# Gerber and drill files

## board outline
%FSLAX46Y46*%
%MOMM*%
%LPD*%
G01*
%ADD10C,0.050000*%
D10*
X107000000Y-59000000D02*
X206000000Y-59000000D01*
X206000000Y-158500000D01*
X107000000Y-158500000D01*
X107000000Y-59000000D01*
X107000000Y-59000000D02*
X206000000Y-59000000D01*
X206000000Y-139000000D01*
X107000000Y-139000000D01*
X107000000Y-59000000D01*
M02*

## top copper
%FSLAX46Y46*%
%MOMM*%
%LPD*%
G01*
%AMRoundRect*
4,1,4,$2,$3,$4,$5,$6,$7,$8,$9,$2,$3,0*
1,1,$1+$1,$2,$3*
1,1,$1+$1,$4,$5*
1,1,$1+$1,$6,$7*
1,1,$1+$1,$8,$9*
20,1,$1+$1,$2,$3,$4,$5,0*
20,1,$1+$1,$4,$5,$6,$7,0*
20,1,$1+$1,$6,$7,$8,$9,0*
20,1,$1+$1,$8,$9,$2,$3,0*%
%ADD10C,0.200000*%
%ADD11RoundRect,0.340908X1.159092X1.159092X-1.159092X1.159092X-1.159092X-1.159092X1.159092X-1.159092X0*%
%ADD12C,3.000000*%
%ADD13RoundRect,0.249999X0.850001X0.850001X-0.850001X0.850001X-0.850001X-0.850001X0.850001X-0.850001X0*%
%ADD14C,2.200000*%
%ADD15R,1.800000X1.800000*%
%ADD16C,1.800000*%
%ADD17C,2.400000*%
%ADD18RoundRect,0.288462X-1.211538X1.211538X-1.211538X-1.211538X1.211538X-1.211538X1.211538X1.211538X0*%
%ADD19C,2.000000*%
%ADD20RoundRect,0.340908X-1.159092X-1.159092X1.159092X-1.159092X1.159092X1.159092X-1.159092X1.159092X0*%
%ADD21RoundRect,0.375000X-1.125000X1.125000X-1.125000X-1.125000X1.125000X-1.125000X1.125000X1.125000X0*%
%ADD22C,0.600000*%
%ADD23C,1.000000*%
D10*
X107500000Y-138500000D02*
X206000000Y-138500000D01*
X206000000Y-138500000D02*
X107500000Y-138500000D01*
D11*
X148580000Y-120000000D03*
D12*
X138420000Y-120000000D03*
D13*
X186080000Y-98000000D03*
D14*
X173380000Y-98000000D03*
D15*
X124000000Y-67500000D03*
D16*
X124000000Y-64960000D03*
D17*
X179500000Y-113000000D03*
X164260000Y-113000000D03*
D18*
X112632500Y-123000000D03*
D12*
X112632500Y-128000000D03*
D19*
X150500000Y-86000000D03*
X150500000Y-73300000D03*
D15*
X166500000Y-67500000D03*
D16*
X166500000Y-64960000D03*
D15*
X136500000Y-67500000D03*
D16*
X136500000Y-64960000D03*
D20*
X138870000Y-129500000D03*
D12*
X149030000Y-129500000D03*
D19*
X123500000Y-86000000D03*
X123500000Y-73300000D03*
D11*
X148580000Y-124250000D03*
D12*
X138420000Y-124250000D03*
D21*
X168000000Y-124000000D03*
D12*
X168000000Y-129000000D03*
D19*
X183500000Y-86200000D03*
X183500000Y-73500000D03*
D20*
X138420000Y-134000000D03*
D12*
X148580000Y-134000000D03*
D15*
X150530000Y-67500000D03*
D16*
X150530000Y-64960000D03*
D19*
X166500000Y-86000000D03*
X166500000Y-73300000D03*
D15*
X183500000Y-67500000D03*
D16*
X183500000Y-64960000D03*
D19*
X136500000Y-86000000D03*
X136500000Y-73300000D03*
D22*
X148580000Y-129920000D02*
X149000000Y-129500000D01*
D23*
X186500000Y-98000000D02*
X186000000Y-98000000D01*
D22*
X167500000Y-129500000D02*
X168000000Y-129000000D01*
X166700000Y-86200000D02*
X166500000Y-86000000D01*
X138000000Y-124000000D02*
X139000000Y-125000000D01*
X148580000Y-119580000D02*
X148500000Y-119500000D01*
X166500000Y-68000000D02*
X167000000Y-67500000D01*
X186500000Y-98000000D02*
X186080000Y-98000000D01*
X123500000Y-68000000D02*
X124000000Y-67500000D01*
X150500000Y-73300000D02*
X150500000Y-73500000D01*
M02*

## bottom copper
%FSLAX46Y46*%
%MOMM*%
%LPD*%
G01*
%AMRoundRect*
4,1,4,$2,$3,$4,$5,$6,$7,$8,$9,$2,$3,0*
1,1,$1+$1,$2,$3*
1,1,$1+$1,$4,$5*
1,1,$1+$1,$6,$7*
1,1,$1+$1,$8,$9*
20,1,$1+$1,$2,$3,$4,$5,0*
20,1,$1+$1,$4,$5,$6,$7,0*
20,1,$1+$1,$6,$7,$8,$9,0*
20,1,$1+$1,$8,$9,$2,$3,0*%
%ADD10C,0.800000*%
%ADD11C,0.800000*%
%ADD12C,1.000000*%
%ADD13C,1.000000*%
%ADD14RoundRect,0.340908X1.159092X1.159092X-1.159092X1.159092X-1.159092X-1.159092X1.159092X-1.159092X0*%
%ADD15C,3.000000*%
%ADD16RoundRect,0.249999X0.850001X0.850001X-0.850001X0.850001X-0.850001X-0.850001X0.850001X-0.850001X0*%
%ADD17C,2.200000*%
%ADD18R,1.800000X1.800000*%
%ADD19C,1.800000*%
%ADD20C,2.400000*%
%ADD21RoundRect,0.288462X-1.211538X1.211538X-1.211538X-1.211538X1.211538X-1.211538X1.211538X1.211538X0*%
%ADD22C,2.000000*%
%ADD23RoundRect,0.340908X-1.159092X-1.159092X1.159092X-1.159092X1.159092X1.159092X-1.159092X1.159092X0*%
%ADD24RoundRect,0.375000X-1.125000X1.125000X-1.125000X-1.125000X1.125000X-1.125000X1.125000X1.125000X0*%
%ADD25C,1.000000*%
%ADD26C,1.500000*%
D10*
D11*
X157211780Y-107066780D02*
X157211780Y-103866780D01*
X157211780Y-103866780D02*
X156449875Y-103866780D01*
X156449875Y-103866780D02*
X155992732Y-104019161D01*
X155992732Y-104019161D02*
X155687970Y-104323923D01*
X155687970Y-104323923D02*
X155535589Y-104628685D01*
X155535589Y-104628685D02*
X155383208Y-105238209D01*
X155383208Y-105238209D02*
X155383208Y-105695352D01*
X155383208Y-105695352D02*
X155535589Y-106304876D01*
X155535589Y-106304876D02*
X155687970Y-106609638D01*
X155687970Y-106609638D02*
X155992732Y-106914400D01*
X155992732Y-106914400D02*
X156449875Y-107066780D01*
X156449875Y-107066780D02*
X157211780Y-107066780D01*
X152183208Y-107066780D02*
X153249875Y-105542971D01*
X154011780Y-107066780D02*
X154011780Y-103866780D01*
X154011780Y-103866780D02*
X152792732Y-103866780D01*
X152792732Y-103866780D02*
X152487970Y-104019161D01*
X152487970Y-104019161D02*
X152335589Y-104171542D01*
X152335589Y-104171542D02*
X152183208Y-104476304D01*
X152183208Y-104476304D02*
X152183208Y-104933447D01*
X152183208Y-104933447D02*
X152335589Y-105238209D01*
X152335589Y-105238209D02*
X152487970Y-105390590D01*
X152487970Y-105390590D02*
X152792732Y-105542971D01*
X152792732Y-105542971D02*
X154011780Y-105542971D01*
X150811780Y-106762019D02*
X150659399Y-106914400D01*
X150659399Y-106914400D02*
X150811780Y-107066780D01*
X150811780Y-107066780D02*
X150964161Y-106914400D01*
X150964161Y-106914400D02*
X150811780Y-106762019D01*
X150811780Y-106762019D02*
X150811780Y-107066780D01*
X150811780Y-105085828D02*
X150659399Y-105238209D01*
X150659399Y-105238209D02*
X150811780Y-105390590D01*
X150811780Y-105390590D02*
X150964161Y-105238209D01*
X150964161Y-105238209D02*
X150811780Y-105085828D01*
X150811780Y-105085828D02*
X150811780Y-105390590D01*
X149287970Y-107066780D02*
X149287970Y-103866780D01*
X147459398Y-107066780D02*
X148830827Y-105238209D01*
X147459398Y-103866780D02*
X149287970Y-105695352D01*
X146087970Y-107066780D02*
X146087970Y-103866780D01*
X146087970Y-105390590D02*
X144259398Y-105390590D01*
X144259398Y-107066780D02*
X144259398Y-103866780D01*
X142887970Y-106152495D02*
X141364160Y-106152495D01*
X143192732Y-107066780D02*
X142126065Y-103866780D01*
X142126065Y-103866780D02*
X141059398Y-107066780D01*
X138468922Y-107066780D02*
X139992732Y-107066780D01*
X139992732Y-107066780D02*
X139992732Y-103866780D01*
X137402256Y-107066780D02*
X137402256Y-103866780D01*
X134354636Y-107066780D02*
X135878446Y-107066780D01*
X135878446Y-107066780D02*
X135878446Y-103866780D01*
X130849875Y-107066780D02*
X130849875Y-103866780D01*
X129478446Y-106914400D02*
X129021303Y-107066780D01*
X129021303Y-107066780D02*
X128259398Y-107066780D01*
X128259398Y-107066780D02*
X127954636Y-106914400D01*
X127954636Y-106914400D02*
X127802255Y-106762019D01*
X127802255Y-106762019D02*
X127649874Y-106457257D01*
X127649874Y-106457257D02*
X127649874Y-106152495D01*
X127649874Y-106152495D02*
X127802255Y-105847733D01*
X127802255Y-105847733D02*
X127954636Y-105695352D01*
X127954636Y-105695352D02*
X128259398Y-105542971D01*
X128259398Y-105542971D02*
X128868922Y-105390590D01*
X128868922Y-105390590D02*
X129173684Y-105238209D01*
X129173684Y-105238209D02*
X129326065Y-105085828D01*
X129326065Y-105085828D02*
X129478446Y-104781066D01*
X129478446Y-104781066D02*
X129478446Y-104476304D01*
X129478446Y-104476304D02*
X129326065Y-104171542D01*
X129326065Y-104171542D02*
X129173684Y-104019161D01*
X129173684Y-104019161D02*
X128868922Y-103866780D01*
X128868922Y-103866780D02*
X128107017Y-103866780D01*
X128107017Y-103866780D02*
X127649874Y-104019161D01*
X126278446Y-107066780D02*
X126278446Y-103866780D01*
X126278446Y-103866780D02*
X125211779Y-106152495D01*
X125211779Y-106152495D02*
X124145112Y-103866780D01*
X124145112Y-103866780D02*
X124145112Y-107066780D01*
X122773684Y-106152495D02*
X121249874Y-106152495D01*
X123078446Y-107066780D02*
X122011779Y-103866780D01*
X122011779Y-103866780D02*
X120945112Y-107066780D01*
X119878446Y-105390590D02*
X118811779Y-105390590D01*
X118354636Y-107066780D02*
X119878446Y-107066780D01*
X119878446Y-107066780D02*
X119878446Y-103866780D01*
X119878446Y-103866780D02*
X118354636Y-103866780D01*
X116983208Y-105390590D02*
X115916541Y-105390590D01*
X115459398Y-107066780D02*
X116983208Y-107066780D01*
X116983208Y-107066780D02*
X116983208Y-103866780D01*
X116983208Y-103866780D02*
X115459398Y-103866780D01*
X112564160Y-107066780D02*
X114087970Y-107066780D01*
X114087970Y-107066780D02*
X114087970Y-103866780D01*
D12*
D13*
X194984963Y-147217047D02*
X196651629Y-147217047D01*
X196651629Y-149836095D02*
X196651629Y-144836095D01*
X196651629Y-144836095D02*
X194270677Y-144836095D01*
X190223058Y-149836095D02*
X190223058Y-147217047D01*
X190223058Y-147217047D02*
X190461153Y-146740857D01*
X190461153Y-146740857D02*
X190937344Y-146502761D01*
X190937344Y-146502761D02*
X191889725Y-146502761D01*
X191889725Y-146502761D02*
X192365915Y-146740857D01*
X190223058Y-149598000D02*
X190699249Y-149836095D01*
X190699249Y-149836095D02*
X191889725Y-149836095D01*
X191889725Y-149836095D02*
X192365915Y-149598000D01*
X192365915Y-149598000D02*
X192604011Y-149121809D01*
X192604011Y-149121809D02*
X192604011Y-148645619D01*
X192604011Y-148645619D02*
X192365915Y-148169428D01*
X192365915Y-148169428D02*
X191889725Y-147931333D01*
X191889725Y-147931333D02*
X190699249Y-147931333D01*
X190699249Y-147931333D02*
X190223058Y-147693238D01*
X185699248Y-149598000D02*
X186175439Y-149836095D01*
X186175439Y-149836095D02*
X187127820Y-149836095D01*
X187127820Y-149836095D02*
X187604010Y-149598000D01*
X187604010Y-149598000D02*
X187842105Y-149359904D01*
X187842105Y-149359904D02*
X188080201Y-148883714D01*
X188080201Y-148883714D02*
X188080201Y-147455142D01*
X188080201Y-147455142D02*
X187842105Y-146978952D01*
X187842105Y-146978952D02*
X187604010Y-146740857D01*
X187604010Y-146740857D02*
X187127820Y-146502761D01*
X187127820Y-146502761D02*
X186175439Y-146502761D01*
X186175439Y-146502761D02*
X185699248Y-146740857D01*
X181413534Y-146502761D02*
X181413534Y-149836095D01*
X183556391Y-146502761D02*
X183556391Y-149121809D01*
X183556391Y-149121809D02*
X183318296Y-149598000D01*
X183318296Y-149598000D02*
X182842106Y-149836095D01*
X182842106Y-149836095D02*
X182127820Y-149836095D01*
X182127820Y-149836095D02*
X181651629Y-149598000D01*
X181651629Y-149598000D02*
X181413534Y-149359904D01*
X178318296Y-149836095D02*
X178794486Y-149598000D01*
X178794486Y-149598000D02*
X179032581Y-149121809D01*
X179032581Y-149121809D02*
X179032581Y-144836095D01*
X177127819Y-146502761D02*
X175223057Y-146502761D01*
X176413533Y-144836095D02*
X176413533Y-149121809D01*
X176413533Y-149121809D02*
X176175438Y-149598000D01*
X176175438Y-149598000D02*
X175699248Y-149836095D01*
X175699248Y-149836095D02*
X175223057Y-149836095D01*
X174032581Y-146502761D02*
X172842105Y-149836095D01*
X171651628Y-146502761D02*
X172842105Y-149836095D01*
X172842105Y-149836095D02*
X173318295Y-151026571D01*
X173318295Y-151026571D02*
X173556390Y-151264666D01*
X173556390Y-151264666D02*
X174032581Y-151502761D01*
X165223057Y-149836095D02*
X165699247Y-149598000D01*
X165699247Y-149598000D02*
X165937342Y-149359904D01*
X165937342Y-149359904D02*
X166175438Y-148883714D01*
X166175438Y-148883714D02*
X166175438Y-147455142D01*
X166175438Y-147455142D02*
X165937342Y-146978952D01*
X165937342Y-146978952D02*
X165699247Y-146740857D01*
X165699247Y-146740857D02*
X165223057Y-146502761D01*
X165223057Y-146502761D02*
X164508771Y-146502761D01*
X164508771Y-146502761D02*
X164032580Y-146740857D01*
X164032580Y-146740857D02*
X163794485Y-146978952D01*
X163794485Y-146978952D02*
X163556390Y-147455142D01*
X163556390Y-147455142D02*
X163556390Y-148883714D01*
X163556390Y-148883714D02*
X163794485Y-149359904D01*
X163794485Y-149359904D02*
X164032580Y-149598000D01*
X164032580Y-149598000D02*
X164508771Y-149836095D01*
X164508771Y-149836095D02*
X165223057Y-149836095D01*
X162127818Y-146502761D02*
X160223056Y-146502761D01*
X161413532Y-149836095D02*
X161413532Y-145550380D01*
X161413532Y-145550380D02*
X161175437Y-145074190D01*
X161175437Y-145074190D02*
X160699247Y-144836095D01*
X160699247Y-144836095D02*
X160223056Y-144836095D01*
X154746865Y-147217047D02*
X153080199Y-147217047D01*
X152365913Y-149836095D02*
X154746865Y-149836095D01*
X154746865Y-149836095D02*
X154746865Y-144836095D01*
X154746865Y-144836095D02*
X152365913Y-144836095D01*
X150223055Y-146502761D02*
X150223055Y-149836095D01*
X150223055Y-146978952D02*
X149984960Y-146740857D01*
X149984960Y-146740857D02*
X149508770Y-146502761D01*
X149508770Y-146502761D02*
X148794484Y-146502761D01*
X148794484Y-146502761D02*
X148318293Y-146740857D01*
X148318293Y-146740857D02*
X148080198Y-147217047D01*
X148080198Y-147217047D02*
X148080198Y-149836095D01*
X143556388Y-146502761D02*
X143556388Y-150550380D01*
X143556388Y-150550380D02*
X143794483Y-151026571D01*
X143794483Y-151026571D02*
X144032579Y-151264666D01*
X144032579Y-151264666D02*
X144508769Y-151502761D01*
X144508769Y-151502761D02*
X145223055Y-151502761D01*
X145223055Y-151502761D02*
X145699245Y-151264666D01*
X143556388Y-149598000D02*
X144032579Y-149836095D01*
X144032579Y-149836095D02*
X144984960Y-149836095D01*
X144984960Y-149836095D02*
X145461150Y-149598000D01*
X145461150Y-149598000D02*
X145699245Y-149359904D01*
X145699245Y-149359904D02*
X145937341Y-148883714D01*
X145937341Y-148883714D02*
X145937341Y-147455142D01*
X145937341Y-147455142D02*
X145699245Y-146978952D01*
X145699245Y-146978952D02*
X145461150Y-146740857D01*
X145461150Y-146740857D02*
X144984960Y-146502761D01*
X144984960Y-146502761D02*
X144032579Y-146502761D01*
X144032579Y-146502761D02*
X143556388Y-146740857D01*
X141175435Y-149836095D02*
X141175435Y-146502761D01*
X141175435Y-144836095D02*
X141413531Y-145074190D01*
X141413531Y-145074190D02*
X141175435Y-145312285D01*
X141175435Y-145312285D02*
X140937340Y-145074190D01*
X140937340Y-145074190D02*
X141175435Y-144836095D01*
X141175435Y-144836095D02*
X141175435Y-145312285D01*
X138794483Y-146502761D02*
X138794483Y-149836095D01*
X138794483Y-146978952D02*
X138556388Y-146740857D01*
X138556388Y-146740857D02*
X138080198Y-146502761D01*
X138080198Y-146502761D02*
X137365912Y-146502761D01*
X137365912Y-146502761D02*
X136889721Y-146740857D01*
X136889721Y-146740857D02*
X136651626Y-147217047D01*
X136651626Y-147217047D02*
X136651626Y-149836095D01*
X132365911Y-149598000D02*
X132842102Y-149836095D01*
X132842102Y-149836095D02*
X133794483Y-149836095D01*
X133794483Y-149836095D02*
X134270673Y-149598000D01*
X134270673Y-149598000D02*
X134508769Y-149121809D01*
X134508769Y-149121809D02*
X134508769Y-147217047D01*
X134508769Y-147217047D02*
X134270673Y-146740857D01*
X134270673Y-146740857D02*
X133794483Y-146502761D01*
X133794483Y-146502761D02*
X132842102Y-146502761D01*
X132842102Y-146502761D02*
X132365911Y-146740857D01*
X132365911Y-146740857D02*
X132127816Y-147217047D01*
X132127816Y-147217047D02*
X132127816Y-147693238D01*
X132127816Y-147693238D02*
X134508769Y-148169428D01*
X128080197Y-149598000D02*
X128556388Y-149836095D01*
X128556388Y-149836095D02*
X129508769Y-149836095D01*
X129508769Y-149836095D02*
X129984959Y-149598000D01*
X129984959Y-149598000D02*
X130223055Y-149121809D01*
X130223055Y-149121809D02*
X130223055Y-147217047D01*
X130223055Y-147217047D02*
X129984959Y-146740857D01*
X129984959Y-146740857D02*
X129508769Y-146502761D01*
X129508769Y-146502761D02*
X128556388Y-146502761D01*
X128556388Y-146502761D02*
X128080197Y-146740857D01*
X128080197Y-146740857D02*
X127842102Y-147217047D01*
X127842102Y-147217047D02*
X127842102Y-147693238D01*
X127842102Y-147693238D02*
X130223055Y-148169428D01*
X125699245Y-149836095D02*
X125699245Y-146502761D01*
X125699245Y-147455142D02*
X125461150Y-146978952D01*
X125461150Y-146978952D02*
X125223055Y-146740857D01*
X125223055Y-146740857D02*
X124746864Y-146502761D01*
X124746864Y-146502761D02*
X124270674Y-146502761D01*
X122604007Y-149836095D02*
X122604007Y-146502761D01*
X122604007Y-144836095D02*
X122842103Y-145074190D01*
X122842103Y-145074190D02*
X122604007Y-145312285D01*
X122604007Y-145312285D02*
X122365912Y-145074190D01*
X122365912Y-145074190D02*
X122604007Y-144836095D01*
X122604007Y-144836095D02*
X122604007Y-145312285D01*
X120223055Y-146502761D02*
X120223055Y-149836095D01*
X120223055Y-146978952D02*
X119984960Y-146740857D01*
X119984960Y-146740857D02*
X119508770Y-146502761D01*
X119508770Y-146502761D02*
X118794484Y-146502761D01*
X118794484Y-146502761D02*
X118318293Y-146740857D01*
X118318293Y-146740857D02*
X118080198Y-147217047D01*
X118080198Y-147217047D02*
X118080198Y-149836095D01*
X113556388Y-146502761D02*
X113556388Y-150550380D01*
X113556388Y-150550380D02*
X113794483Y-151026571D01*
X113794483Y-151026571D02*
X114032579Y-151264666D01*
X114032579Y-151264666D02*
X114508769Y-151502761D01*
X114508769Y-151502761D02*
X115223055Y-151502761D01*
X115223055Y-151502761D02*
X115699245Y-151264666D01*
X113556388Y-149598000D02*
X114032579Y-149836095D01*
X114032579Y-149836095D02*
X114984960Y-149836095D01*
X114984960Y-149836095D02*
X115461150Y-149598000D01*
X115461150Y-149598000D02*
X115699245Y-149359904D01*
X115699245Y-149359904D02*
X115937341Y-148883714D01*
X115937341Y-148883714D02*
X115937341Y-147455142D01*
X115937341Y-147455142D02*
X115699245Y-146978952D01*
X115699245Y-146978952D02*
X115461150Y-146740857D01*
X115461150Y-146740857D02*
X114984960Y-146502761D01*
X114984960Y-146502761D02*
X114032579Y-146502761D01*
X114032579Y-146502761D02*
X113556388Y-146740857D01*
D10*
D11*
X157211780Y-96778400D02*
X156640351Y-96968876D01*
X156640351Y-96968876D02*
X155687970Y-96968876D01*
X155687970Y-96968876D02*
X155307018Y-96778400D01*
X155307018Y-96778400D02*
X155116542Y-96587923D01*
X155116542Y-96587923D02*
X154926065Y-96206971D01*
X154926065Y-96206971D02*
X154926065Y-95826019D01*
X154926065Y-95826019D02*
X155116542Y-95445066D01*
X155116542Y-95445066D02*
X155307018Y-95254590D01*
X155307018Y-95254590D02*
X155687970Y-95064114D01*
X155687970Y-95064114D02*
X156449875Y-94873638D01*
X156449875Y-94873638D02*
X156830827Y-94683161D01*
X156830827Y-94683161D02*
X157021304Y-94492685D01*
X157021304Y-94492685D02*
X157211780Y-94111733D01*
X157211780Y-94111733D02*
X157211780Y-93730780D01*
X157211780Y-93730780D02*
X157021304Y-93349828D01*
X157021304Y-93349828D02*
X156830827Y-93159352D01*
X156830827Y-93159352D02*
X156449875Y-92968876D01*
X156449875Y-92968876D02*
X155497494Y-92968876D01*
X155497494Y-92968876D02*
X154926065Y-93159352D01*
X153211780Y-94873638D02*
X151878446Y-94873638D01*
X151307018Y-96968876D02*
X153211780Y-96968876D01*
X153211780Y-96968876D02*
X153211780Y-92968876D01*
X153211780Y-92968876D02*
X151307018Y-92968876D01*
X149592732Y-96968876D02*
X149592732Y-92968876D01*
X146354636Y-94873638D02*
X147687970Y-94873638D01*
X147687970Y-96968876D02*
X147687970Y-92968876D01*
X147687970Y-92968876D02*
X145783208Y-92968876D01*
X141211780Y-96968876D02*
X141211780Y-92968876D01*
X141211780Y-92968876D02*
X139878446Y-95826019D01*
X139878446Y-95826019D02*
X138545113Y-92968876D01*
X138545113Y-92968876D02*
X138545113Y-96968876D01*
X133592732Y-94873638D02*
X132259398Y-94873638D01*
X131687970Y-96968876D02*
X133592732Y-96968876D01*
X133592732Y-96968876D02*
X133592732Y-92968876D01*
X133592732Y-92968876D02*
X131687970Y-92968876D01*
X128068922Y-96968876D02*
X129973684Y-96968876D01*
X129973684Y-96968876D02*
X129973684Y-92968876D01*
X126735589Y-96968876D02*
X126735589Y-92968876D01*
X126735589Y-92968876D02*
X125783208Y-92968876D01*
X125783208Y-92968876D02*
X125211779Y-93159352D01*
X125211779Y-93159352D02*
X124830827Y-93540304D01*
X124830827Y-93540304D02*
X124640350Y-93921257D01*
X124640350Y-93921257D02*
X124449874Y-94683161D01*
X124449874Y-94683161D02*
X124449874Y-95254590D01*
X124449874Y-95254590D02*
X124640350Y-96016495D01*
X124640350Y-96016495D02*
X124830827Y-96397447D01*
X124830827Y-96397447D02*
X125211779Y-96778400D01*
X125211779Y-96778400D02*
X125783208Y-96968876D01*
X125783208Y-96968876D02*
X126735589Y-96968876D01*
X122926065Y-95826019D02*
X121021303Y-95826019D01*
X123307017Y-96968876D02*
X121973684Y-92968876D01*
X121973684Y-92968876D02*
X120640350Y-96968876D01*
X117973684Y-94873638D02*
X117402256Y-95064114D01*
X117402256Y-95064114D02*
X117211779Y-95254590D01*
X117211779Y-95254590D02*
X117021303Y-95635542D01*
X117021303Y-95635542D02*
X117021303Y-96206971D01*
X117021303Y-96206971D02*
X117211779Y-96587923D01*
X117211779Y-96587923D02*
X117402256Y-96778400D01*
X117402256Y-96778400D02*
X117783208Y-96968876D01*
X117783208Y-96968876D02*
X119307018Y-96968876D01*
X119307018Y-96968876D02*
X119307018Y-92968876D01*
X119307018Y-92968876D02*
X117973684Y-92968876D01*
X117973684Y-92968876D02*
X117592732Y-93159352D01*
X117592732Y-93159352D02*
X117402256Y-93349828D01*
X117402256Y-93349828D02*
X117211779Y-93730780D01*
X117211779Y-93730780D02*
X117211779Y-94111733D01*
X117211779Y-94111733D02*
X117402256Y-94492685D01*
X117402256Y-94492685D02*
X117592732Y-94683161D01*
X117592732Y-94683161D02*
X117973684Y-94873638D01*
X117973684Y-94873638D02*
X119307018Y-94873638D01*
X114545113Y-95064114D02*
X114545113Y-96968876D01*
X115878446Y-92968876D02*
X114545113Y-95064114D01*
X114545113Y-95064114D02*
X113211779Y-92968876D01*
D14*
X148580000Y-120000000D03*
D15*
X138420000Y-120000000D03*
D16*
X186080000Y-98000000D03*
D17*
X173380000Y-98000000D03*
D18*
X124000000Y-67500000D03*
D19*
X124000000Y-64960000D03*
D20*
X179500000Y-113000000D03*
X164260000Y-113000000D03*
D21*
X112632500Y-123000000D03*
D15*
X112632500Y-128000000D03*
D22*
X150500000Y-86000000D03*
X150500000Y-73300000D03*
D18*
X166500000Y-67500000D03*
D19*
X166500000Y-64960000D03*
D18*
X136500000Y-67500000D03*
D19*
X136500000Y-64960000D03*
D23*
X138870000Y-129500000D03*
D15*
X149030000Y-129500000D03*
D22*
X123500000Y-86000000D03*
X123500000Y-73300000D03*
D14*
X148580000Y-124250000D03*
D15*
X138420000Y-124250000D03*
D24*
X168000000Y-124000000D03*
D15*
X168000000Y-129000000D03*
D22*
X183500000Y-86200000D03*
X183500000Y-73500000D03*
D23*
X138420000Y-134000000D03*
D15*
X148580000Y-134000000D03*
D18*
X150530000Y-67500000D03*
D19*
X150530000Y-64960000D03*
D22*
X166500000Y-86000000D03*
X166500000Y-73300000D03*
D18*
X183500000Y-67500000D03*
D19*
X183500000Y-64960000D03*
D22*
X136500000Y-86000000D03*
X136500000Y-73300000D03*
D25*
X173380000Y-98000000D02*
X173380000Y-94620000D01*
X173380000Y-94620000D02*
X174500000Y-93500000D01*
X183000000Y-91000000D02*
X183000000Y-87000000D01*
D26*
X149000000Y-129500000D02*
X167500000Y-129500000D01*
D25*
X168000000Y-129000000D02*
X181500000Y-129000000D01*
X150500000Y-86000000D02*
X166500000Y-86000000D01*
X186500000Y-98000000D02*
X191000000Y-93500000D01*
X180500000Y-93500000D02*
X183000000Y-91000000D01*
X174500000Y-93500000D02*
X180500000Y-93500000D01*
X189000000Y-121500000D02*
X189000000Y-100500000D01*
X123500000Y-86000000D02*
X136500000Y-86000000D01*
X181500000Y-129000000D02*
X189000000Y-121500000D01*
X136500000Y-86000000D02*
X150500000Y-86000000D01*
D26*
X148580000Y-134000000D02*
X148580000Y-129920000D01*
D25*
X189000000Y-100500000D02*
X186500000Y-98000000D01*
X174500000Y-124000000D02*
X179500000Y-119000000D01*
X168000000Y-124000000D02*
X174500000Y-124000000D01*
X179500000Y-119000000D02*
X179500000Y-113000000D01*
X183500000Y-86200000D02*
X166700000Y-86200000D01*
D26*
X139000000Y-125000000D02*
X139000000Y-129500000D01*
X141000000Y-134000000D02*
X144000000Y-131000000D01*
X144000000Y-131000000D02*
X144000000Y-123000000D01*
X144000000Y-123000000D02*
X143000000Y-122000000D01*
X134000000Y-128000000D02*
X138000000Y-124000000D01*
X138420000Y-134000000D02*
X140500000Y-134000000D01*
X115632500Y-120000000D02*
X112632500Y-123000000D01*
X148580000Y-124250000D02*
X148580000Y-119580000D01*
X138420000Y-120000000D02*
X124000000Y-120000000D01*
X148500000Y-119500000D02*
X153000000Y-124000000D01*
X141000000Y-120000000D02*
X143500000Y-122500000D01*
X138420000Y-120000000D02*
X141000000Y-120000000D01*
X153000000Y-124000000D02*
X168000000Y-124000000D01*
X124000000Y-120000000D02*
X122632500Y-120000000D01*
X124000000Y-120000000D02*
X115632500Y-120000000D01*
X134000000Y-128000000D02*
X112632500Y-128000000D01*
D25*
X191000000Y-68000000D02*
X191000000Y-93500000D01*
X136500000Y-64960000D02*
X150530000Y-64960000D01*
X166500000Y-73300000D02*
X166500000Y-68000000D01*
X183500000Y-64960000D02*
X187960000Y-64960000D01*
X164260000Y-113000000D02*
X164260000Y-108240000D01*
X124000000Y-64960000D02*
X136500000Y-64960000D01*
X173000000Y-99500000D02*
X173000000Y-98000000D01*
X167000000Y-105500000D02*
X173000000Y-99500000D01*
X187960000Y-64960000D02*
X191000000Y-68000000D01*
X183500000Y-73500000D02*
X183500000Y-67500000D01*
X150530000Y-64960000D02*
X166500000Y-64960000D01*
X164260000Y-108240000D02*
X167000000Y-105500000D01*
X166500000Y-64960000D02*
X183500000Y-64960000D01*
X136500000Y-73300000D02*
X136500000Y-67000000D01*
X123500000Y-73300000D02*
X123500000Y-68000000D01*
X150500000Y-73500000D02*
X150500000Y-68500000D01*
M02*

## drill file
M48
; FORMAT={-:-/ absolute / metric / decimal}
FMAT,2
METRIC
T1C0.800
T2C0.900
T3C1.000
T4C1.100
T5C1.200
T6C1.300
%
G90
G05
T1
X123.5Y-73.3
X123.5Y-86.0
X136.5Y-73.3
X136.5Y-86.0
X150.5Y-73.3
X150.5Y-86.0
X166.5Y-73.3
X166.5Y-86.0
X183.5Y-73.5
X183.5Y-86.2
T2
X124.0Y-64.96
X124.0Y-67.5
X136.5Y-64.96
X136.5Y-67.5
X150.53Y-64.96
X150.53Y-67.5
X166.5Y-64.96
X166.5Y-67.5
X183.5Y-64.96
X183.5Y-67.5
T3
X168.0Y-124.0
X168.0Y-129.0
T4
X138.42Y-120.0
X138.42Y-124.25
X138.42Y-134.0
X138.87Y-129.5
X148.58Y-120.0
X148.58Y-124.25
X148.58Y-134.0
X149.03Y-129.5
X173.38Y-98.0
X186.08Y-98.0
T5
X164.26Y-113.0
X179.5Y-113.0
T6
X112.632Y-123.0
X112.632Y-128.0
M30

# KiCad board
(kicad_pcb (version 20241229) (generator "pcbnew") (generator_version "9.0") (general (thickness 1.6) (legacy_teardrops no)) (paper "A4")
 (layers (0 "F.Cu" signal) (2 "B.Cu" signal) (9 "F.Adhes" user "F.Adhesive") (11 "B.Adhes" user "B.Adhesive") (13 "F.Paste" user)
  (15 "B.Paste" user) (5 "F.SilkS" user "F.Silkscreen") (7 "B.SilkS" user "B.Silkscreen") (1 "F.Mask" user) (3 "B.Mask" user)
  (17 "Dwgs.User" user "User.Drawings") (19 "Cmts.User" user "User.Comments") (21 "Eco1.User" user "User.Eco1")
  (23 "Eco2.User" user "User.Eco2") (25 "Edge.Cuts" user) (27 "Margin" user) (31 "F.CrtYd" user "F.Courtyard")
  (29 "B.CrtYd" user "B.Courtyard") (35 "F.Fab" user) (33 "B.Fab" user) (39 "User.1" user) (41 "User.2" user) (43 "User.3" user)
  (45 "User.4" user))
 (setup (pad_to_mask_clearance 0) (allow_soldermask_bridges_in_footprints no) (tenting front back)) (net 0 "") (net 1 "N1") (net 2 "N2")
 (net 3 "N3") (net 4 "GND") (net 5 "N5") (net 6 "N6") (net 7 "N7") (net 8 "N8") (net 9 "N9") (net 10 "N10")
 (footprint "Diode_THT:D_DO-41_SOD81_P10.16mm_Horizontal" (layer "F.Cu") (at 148.58 120 180)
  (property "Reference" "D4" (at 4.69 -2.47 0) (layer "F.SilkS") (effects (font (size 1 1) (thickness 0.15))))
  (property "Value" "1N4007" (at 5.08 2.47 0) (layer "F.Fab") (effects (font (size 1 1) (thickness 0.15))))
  (pad "1" thru_hole roundrect (at 0 0 180) (size 3 3) (drill 1.1) (layers "*.Cu" "*.Mask") (remove_unused_layers no)
   (roundrect_rratio 0.113636) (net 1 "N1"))
  (pad "2" thru_hole circle (at 10.16 0 180) (size 3 3) (drill 1.1) (layers "*.Cu" "*.Mask") (remove_unused_layers no) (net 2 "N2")))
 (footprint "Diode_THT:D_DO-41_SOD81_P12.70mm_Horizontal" (layer "F.Cu") (at 186.08 98 180)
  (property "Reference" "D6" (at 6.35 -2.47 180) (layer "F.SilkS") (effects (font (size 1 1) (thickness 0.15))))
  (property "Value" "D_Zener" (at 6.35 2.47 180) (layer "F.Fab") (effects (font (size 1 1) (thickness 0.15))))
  (pad "1" thru_hole roundrect (at 0 0 180) (size 2.2 2.2) (drill 1.1) (layers "*.Cu" "*.Mask") (remove_unused_layers no)
   (roundrect_rratio 0.113636) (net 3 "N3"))
  (pad "2" thru_hole circle (at 12.7 0 180) (size 2.2 2.2) (drill 1.1) (layers "*.Cu" "*.Mask") (remove_unused_layers no) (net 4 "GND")))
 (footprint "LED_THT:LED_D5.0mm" (layer "F.Cu") (at 124 67.5 90)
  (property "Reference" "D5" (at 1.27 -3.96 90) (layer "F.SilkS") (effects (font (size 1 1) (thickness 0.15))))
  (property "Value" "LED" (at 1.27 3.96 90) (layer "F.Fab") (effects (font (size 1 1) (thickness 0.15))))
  (pad "1" thru_hole rect (at 0 0 90) (size 1.8 1.8) (drill 0.9) (layers "*.Cu" "*.Mask") (remove_unused_layers no) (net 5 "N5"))
  (pad "2" thru_hole circle (at 2.54 0 90) (size 1.8 1.8) (drill 0.9) (layers "*.Cu" "*.Mask") (remove_unused_layers no) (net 3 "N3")))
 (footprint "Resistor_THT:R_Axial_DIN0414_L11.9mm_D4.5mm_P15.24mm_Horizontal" (layer "F.Cu") (at 179.5 113 180)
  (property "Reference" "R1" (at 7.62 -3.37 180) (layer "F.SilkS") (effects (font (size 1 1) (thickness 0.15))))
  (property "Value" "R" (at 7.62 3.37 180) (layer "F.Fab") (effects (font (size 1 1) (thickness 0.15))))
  (pad "1" thru_hole circle (at 0 0 180) (size 2.4 2.4) (drill 1.2) (layers "*.Cu" "*.Mask") (remove_unused_layers no) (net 1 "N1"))
  (pad "2" thru_hole circle (at 15.24 0 180) (size 2.4 2.4) (drill 1.2) (layers "*.Cu" "*.Mask") (remove_unused_layers no) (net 3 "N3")))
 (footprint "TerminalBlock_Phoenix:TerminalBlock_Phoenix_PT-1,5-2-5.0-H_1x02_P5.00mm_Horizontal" (layer "F.Cu") (at 112.6325 123 -90)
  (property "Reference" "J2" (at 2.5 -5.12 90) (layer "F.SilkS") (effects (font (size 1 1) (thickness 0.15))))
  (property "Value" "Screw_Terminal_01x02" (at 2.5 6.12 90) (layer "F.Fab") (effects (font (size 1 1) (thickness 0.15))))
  (pad "1" thru_hole roundrect (at 0 0 270) (size 3 3) (drill 1.3) (layers "*.Cu" "*.Mask") (remove_unused_layers no)
   (roundrect_rratio 0.096154) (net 2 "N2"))
  (pad "2" thru_hole circle (at 5 0 270) (size 3 3) (drill 1.3) (layers "*.Cu" "*.Mask") (remove_unused_layers no) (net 3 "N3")))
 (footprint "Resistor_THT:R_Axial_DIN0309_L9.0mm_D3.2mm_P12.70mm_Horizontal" (layer "F.Cu") (at 150.5 86 90)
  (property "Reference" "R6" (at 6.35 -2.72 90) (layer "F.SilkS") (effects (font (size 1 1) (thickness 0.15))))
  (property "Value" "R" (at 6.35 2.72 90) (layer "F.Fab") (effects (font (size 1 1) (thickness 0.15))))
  (pad "1" thru_hole circle (at 0 0 90) (size 2 2) (drill 0.8) (layers "*.Cu" "*.Mask") (remove_unused_layers no) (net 4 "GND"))
  (pad "2" thru_hole circle (at 12.7 0 90) (size 2 2) (drill 0.8) (layers "*.Cu" "*.Mask") (remove_unused_layers no) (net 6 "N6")))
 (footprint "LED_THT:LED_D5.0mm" (layer "F.Cu") (at 166.5 67.5 90)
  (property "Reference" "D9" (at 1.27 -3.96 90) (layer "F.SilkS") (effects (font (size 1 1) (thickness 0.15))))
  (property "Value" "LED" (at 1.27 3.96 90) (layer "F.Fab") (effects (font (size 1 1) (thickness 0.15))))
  (pad "1" thru_hole rect (at 0 0 90) (size 1.8 1.8) (drill 0.9) (layers "*.Cu" "*.Mask") (remove_unused_layers no) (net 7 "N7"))
  (pad "2" thru_hole circle (at 2.54 0 90) (size 1.8 1.8) (drill 0.9) (layers "*.Cu" "*.Mask") (remove_unused_layers no) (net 3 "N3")))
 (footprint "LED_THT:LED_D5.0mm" (layer "F.Cu") (at 136.5 67.5 90)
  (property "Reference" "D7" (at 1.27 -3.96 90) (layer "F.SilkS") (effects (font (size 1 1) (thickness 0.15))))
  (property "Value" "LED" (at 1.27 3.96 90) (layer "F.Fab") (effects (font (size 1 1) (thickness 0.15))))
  (pad "1" thru_hole rect (at 0 0 90) (size 1.8 1.8) (drill 0.9) (layers "*.Cu" "*.Mask") (remove_unused_layers no) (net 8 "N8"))
  (pad "2" thru_hole circle (at 2.54 0 90) (size 1.8 1.8) (drill 0.9) (layers "*.Cu" "*.Mask") (remove_unused_layers no) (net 3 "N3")))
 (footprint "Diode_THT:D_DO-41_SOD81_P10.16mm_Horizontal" (layer "F.Cu") (at 138.87 129.5)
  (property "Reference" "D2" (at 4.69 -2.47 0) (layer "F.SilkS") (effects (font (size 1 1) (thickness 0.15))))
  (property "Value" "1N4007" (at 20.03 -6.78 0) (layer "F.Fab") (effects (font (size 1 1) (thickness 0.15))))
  (pad "1" thru_hole roundrect (at 0 0) (size 3 3) (drill 1.1) (layers "*.Cu" "*.Mask") (remove_unused_layers no)
   (roundrect_rratio 0.113636) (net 1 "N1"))
  (pad "2" thru_hole circle (at 10.16 0) (size 3 3) (drill 1.1) (layers "*.Cu" "*.Mask") (remove_unused_layers no) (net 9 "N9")))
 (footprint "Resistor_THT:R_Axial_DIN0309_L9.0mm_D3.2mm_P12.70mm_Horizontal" (layer "F.Cu") (at 123.5 86 90)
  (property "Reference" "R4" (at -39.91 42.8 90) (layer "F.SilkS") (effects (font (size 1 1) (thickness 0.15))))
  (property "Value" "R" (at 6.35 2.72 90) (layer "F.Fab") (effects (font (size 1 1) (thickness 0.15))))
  (pad "1" thru_hole circle (at 0 0 90) (size 2 2) (drill 0.8) (layers "*.Cu" "*.Mask") (remove_unused_layers no) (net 4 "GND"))
  (pad "2" thru_hole circle (at 12.7 0 90) (size 2 2) (drill 0.8) (layers "*.Cu" "*.Mask") (remove_unused_layers no) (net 8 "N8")))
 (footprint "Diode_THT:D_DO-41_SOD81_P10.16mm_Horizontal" (layer "F.Cu") (at 148.58 124.25 180)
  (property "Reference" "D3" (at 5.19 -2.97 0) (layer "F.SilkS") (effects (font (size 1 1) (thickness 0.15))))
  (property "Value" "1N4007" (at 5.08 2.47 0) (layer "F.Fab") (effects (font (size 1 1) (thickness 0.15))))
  (pad "1" thru_hole roundrect (at 0 0 180) (size 3 3) (drill 1.1) (layers "*.Cu" "*.Mask") (remove_unused_layers no)
   (roundrect_rratio 0.113636) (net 2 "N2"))
  (pad "2" thru_hole circle (at 10.16 0 180) (size 3 3) (drill 1.1) (layers "*.Cu" "*.Mask") (remove_unused_layers no) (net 4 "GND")))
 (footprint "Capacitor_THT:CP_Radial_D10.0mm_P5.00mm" (layer "F.Cu") (at 168 124 -90)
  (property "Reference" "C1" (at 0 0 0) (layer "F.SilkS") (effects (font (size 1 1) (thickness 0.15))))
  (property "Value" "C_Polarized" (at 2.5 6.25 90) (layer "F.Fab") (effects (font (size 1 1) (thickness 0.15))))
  (pad "1" thru_hole roundrect (at 0 0 270) (size 3 3) (drill 1) (layers "*.Cu" "*.Mask") (remove_unused_layers no) (roundrect_rratio 0.125)
   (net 1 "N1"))
  (pad "2" thru_hole circle (at 5 0 270) (size 3 3) (drill 1) (layers "*.Cu" "*.Mask") (remove_unused_layers no) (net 4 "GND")))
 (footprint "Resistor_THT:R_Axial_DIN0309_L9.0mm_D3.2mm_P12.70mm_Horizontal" (layer "F.Cu") (at 183.5 86.2 90)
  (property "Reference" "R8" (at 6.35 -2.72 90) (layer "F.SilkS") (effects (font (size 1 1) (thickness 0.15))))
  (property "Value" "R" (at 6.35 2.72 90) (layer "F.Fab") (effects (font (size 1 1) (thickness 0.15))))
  (pad "1" thru_hole circle (at 0 0 90) (size 2 2) (drill 0.8) (layers "*.Cu" "*.Mask") (remove_unused_layers no) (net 1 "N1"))
  (pad "2" thru_hole circle (at 12.7 0 90) (size 2 2) (drill 0.8) (layers "*.Cu" "*.Mask") (remove_unused_layers no) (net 3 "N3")))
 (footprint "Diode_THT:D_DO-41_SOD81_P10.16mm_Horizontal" (layer "F.Cu") (at 138.42 134)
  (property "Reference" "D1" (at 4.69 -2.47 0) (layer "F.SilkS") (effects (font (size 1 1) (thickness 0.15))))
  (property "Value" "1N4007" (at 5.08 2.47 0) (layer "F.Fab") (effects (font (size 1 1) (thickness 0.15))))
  (pad "1" thru_hole roundrect (at 0 0) (size 3 3) (drill 1.1) (layers "*.Cu" "*.Mask") (remove_unused_layers no)
   (roundrect_rratio 0.113636) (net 9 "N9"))
  (pad "2" thru_hole circle (at 10.16 0) (size 3 3) (drill 1.1) (layers "*.Cu" "*.Mask") (remove_unused_layers no) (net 4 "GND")))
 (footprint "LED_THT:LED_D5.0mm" (layer "F.Cu") (at 150.53 67.5 90)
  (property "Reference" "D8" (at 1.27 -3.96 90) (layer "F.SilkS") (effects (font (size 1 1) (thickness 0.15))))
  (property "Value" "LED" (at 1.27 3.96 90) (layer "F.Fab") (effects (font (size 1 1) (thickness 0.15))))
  (pad "1" thru_hole rect (at 0 0 90) (size 1.8 1.8) (drill 0.9) (layers "*.Cu" "*.Mask") (remove_unused_layers no) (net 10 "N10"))
  (pad "2" thru_hole circle (at 2.54 0 90) (size 1.8 1.8) (drill 0.9) (layers "*.Cu" "*.Mask") (remove_unused_layers no) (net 3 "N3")))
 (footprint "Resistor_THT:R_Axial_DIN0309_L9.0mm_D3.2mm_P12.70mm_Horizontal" (layer "F.Cu") (at 166.5 86 90)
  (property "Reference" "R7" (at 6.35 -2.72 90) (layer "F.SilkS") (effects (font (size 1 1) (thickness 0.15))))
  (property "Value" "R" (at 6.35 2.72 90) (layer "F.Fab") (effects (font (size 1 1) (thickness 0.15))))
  (pad "1" thru_hole circle (at 0 0 90) (size 2 2) (drill 0.8) (layers "*.Cu" "*.Mask") (remove_unused_layers no) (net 1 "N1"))
  (pad "2" thru_hole circle (at 12.7 0 90) (size 2 2) (drill 0.8) (layers "*.Cu" "*.Mask") (remove_unused_layers no) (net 3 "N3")))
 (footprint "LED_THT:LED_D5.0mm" (layer "F.Cu") (at 183.5 67.5 90)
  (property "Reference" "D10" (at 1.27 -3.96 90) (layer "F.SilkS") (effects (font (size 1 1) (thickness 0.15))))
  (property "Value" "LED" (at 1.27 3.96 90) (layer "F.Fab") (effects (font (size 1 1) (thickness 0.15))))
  (pad "1" thru_hole rect (at 0 0 90) (size 1.8 1.8) (drill 0.9) (layers "*.Cu" "*.Mask") (remove_unused_layers no) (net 6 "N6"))
  (pad "2" thru_hole circle (at 2.54 0 90) (size 1.8 1.8) (drill 0.9) (layers "*.Cu" "*.Mask") (remove_unused_layers no) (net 3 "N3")))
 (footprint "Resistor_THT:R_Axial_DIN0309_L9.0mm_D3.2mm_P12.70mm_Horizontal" (layer "F.Cu") (at 136.5 86 90)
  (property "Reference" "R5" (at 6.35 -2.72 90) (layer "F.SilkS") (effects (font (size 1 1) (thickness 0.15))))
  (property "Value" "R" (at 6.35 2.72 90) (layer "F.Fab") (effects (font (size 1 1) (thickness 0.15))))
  (pad "1" thru_hole circle (at 0 0 90) (size 2 2) (drill 0.8) (layers "*.Cu" "*.Mask") (remove_unused_layers no) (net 4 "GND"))
  (pad "2" thru_hole circle (at 12.7 0 90) (size 2 2) (drill 0.8) (layers "*.Cu" "*.Mask") (remove_unused_layers no) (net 5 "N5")))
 (gr_line (start 107.5 138.5) (end 206 138.5) (stroke (width 0.2) (type default)) (layer "F.Cu"))
 (gr_line (start 206 138.5) (end 107.5 138.5) (stroke (width 0.2) (type default)) (layer "F.Cu"))
 (gr_rect (start 107 59) (end 206 158.5) (stroke (width 0.05) (type default)) (fill no) (layer "Edge.Cuts"))
 (gr_rect (start 107 59) (end 206 139) (stroke (width 0.05) (type default)) (fill no) (layer "Edge.Cuts"))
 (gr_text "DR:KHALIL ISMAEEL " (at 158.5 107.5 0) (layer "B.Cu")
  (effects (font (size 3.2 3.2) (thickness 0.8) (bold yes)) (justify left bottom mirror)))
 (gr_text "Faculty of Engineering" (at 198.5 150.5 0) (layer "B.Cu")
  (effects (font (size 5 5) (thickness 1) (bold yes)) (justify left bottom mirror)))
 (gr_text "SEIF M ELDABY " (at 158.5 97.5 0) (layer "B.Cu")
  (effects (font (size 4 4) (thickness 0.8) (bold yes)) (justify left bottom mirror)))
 (segment (start 148.58 129.92) (end 149 129.5) (width 0.6) (layer "F.Cu") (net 4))
 (segment (start 186.5 98) (end 186 98) (width 1) (layer "F.Cu") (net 4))
 (segment (start 167.5 129.5) (end 168 129) (width 0.6) (layer "F.Cu") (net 4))
 (segment (start 173.38 98) (end 173.38 94.62) (width 1) (layer "B.Cu") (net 4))
 (segment (start 173.38 94.62) (end 174.5 93.5) (width 1) (layer "B.Cu") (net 4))
 (segment (start 183 91) (end 183 87) (width 1) (layer "B.Cu") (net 4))
 (segment (start 149 129.5) (end 167.5 129.5) (width 1.5) (layer "B.Cu") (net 4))
 (segment (start 168 129) (end 181.5 129) (width 1) (layer "B.Cu") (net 4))
 (segment (start 150.5 86) (end 166.5 86) (width 1) (layer "B.Cu") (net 4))
 (segment (start 186.5 98) (end 191 93.5) (width 1) (layer "B.Cu") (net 4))
 (segment (start 180.5 93.5) (end 183 91) (width 1) (layer "B.Cu") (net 4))
 (segment (start 174.5 93.5) (end 180.5 93.5) (width 1) (layer "B.Cu") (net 4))
 (segment (start 189 121.5) (end 189 100.5) (width 1) (layer "B.Cu") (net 4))
 (segment (start 123.5 86) (end 136.5 86) (width 1) (layer "B.Cu") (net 4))
 (segment (start 181.5 129) (end 189 121.5) (width 1) (layer "B.Cu") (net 4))
 (segment (start 136.5 86) (end 150.5 86) (width 1) (layer "B.Cu") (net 4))
 (segment (start 148.58 134) (end 148.58 129.92) (width 1.5) (layer "B.Cu") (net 4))
 (segment (start 189 100.5) (end 186.5 98) (width 1) (layer "B.Cu") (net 4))
 (segment (start 166.7 86.2) (end 166.5 86) (width 0.6) (layer "F.Cu") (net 1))
 (segment (start 174.5 124) (end 179.5 119) (width 1) (layer "B.Cu") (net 1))
 (segment (start 168 124) (end 174.5 124) (width 1) (layer "B.Cu") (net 1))
 (segment (start 179.5 119) (end 179.5 113) (width 1) (layer "B.Cu") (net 1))
 (segment (start 183.5 86.2) (end 166.7 86.2) (width 1) (layer "B.Cu") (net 1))
 (segment (start 138 124) (end 139 125) (width 0.6) (layer "F.Cu") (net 9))
 (segment (start 139 125) (end 139 129.5) (width 1.5) (layer "B.Cu") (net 9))
 (segment (start 141 134) (end 144 131) (width 1.5) (layer "B.Cu") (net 9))
 (segment (start 144 131) (end 144 123) (width 1.5) (layer "B.Cu") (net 9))
 (segment (start 144 123) (end 143 122) (width 1.5) (layer "B.Cu") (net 9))
 (segment (start 134 128) (end 138 124) (width 1.5) (layer "B.Cu") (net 9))
 (segment (start 138.42 134) (end 140.5 134) (width 1.5) (layer "B.Cu") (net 9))
 (segment (start 148.58 119.58) (end 148.5 119.5) (width 0.6) (layer "F.Cu") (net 2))
 (segment (start 115.6325 120) (end 112.6325 123) (width 1.5) (layer "B.Cu") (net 2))
 (segment (start 148.58 124.25) (end 148.58 119.58) (width 1.5) (layer "B.Cu") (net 2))
 (segment (start 138.42 120) (end 124 120) (width 1.5) (layer "B.Cu") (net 2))
 (segment (start 148.5 119.5) (end 153 124) (width 1.5) (layer "B.Cu") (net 2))
 (segment (start 141 120) (end 143.5 122.5) (width 1.5) (layer "B.Cu") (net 2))
 (segment (start 138.42 120) (end 141 120) (width 1.5) (layer "B.Cu") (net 2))
 (segment (start 153 124) (end 168 124) (width 1.5) (layer "B.Cu") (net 2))
 (segment (start 124 120) (end 122.6325 120) (width 1.5) (layer "B.Cu") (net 2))
 (segment (start 124 120) (end 115.6325 120) (width 1.5) (layer "B.Cu") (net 2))
 (segment (start 166.5 68) (end 167 67.5) (width 0.6) (layer "F.Cu") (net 3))
 (segment (start 186.5 98) (end 186.08 98) (width 0.6) (layer "F.Cu") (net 3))
 (segment (start 134 128) (end 112.6325 128) (width 1.5) (layer "B.Cu") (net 3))
 (segment (start 191 68) (end 191 93.5) (width 1) (layer "B.Cu") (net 3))
 (segment (start 136.5 64.96) (end 150.53 64.96) (width 1) (layer "B.Cu") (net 3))
 (segment (start 166.5 73.3) (end 166.5 68) (width 1) (layer "B.Cu") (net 3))
 (segment (start 183.5 64.96) (end 187.96 64.96) (width 1) (layer "B.Cu") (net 3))
 (segment (start 164.26 113) (end 164.26 108.24) (width 1) (layer "B.Cu") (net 3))
 (segment (start 124 64.96) (end 136.5 64.96) (width 1) (layer "B.Cu") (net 3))
 (segment (start 173 99.5) (end 173 98) (width 1) (layer "B.Cu") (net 3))
 (segment (start 167 105.5) (end 173 99.5) (width 1) (layer "B.Cu") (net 3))
 (segment (start 187.96 64.96) (end 191 68) (width 1) (layer "B.Cu") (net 3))
 (segment (start 183.5 73.5) (end 183.5 67.5) (width 1) (layer "B.Cu") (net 3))
 (segment (start 150.53 64.96) (end 166.5 64.96) (width 1) (layer "B.Cu") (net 3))
 (segment (start 164.26 108.24) (end 167 105.5) (width 1) (layer "B.Cu") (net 3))
 (segment (start 166.5 64.96) (end 183.5 64.96) (width 1) (layer "B.Cu") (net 3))
 (segment (start 136.5 73.3) (end 136.5 67) (width 1) (layer "B.Cu") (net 5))
 (segment (start 123.5 68) (end 124 67.5) (width 0.6) (layer "F.Cu") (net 8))
 (segment (start 123.5 73.3) (end 123.5 68) (width 1) (layer "B.Cu") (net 8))
 (segment (start 150.5 73.3) (end 150.5 73.5) (width 0.6) (layer "F.Cu") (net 6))
 (segment (start 150.5 73.5) (end 150.5 68.5) (width 1) (layer "B.Cu") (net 6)))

